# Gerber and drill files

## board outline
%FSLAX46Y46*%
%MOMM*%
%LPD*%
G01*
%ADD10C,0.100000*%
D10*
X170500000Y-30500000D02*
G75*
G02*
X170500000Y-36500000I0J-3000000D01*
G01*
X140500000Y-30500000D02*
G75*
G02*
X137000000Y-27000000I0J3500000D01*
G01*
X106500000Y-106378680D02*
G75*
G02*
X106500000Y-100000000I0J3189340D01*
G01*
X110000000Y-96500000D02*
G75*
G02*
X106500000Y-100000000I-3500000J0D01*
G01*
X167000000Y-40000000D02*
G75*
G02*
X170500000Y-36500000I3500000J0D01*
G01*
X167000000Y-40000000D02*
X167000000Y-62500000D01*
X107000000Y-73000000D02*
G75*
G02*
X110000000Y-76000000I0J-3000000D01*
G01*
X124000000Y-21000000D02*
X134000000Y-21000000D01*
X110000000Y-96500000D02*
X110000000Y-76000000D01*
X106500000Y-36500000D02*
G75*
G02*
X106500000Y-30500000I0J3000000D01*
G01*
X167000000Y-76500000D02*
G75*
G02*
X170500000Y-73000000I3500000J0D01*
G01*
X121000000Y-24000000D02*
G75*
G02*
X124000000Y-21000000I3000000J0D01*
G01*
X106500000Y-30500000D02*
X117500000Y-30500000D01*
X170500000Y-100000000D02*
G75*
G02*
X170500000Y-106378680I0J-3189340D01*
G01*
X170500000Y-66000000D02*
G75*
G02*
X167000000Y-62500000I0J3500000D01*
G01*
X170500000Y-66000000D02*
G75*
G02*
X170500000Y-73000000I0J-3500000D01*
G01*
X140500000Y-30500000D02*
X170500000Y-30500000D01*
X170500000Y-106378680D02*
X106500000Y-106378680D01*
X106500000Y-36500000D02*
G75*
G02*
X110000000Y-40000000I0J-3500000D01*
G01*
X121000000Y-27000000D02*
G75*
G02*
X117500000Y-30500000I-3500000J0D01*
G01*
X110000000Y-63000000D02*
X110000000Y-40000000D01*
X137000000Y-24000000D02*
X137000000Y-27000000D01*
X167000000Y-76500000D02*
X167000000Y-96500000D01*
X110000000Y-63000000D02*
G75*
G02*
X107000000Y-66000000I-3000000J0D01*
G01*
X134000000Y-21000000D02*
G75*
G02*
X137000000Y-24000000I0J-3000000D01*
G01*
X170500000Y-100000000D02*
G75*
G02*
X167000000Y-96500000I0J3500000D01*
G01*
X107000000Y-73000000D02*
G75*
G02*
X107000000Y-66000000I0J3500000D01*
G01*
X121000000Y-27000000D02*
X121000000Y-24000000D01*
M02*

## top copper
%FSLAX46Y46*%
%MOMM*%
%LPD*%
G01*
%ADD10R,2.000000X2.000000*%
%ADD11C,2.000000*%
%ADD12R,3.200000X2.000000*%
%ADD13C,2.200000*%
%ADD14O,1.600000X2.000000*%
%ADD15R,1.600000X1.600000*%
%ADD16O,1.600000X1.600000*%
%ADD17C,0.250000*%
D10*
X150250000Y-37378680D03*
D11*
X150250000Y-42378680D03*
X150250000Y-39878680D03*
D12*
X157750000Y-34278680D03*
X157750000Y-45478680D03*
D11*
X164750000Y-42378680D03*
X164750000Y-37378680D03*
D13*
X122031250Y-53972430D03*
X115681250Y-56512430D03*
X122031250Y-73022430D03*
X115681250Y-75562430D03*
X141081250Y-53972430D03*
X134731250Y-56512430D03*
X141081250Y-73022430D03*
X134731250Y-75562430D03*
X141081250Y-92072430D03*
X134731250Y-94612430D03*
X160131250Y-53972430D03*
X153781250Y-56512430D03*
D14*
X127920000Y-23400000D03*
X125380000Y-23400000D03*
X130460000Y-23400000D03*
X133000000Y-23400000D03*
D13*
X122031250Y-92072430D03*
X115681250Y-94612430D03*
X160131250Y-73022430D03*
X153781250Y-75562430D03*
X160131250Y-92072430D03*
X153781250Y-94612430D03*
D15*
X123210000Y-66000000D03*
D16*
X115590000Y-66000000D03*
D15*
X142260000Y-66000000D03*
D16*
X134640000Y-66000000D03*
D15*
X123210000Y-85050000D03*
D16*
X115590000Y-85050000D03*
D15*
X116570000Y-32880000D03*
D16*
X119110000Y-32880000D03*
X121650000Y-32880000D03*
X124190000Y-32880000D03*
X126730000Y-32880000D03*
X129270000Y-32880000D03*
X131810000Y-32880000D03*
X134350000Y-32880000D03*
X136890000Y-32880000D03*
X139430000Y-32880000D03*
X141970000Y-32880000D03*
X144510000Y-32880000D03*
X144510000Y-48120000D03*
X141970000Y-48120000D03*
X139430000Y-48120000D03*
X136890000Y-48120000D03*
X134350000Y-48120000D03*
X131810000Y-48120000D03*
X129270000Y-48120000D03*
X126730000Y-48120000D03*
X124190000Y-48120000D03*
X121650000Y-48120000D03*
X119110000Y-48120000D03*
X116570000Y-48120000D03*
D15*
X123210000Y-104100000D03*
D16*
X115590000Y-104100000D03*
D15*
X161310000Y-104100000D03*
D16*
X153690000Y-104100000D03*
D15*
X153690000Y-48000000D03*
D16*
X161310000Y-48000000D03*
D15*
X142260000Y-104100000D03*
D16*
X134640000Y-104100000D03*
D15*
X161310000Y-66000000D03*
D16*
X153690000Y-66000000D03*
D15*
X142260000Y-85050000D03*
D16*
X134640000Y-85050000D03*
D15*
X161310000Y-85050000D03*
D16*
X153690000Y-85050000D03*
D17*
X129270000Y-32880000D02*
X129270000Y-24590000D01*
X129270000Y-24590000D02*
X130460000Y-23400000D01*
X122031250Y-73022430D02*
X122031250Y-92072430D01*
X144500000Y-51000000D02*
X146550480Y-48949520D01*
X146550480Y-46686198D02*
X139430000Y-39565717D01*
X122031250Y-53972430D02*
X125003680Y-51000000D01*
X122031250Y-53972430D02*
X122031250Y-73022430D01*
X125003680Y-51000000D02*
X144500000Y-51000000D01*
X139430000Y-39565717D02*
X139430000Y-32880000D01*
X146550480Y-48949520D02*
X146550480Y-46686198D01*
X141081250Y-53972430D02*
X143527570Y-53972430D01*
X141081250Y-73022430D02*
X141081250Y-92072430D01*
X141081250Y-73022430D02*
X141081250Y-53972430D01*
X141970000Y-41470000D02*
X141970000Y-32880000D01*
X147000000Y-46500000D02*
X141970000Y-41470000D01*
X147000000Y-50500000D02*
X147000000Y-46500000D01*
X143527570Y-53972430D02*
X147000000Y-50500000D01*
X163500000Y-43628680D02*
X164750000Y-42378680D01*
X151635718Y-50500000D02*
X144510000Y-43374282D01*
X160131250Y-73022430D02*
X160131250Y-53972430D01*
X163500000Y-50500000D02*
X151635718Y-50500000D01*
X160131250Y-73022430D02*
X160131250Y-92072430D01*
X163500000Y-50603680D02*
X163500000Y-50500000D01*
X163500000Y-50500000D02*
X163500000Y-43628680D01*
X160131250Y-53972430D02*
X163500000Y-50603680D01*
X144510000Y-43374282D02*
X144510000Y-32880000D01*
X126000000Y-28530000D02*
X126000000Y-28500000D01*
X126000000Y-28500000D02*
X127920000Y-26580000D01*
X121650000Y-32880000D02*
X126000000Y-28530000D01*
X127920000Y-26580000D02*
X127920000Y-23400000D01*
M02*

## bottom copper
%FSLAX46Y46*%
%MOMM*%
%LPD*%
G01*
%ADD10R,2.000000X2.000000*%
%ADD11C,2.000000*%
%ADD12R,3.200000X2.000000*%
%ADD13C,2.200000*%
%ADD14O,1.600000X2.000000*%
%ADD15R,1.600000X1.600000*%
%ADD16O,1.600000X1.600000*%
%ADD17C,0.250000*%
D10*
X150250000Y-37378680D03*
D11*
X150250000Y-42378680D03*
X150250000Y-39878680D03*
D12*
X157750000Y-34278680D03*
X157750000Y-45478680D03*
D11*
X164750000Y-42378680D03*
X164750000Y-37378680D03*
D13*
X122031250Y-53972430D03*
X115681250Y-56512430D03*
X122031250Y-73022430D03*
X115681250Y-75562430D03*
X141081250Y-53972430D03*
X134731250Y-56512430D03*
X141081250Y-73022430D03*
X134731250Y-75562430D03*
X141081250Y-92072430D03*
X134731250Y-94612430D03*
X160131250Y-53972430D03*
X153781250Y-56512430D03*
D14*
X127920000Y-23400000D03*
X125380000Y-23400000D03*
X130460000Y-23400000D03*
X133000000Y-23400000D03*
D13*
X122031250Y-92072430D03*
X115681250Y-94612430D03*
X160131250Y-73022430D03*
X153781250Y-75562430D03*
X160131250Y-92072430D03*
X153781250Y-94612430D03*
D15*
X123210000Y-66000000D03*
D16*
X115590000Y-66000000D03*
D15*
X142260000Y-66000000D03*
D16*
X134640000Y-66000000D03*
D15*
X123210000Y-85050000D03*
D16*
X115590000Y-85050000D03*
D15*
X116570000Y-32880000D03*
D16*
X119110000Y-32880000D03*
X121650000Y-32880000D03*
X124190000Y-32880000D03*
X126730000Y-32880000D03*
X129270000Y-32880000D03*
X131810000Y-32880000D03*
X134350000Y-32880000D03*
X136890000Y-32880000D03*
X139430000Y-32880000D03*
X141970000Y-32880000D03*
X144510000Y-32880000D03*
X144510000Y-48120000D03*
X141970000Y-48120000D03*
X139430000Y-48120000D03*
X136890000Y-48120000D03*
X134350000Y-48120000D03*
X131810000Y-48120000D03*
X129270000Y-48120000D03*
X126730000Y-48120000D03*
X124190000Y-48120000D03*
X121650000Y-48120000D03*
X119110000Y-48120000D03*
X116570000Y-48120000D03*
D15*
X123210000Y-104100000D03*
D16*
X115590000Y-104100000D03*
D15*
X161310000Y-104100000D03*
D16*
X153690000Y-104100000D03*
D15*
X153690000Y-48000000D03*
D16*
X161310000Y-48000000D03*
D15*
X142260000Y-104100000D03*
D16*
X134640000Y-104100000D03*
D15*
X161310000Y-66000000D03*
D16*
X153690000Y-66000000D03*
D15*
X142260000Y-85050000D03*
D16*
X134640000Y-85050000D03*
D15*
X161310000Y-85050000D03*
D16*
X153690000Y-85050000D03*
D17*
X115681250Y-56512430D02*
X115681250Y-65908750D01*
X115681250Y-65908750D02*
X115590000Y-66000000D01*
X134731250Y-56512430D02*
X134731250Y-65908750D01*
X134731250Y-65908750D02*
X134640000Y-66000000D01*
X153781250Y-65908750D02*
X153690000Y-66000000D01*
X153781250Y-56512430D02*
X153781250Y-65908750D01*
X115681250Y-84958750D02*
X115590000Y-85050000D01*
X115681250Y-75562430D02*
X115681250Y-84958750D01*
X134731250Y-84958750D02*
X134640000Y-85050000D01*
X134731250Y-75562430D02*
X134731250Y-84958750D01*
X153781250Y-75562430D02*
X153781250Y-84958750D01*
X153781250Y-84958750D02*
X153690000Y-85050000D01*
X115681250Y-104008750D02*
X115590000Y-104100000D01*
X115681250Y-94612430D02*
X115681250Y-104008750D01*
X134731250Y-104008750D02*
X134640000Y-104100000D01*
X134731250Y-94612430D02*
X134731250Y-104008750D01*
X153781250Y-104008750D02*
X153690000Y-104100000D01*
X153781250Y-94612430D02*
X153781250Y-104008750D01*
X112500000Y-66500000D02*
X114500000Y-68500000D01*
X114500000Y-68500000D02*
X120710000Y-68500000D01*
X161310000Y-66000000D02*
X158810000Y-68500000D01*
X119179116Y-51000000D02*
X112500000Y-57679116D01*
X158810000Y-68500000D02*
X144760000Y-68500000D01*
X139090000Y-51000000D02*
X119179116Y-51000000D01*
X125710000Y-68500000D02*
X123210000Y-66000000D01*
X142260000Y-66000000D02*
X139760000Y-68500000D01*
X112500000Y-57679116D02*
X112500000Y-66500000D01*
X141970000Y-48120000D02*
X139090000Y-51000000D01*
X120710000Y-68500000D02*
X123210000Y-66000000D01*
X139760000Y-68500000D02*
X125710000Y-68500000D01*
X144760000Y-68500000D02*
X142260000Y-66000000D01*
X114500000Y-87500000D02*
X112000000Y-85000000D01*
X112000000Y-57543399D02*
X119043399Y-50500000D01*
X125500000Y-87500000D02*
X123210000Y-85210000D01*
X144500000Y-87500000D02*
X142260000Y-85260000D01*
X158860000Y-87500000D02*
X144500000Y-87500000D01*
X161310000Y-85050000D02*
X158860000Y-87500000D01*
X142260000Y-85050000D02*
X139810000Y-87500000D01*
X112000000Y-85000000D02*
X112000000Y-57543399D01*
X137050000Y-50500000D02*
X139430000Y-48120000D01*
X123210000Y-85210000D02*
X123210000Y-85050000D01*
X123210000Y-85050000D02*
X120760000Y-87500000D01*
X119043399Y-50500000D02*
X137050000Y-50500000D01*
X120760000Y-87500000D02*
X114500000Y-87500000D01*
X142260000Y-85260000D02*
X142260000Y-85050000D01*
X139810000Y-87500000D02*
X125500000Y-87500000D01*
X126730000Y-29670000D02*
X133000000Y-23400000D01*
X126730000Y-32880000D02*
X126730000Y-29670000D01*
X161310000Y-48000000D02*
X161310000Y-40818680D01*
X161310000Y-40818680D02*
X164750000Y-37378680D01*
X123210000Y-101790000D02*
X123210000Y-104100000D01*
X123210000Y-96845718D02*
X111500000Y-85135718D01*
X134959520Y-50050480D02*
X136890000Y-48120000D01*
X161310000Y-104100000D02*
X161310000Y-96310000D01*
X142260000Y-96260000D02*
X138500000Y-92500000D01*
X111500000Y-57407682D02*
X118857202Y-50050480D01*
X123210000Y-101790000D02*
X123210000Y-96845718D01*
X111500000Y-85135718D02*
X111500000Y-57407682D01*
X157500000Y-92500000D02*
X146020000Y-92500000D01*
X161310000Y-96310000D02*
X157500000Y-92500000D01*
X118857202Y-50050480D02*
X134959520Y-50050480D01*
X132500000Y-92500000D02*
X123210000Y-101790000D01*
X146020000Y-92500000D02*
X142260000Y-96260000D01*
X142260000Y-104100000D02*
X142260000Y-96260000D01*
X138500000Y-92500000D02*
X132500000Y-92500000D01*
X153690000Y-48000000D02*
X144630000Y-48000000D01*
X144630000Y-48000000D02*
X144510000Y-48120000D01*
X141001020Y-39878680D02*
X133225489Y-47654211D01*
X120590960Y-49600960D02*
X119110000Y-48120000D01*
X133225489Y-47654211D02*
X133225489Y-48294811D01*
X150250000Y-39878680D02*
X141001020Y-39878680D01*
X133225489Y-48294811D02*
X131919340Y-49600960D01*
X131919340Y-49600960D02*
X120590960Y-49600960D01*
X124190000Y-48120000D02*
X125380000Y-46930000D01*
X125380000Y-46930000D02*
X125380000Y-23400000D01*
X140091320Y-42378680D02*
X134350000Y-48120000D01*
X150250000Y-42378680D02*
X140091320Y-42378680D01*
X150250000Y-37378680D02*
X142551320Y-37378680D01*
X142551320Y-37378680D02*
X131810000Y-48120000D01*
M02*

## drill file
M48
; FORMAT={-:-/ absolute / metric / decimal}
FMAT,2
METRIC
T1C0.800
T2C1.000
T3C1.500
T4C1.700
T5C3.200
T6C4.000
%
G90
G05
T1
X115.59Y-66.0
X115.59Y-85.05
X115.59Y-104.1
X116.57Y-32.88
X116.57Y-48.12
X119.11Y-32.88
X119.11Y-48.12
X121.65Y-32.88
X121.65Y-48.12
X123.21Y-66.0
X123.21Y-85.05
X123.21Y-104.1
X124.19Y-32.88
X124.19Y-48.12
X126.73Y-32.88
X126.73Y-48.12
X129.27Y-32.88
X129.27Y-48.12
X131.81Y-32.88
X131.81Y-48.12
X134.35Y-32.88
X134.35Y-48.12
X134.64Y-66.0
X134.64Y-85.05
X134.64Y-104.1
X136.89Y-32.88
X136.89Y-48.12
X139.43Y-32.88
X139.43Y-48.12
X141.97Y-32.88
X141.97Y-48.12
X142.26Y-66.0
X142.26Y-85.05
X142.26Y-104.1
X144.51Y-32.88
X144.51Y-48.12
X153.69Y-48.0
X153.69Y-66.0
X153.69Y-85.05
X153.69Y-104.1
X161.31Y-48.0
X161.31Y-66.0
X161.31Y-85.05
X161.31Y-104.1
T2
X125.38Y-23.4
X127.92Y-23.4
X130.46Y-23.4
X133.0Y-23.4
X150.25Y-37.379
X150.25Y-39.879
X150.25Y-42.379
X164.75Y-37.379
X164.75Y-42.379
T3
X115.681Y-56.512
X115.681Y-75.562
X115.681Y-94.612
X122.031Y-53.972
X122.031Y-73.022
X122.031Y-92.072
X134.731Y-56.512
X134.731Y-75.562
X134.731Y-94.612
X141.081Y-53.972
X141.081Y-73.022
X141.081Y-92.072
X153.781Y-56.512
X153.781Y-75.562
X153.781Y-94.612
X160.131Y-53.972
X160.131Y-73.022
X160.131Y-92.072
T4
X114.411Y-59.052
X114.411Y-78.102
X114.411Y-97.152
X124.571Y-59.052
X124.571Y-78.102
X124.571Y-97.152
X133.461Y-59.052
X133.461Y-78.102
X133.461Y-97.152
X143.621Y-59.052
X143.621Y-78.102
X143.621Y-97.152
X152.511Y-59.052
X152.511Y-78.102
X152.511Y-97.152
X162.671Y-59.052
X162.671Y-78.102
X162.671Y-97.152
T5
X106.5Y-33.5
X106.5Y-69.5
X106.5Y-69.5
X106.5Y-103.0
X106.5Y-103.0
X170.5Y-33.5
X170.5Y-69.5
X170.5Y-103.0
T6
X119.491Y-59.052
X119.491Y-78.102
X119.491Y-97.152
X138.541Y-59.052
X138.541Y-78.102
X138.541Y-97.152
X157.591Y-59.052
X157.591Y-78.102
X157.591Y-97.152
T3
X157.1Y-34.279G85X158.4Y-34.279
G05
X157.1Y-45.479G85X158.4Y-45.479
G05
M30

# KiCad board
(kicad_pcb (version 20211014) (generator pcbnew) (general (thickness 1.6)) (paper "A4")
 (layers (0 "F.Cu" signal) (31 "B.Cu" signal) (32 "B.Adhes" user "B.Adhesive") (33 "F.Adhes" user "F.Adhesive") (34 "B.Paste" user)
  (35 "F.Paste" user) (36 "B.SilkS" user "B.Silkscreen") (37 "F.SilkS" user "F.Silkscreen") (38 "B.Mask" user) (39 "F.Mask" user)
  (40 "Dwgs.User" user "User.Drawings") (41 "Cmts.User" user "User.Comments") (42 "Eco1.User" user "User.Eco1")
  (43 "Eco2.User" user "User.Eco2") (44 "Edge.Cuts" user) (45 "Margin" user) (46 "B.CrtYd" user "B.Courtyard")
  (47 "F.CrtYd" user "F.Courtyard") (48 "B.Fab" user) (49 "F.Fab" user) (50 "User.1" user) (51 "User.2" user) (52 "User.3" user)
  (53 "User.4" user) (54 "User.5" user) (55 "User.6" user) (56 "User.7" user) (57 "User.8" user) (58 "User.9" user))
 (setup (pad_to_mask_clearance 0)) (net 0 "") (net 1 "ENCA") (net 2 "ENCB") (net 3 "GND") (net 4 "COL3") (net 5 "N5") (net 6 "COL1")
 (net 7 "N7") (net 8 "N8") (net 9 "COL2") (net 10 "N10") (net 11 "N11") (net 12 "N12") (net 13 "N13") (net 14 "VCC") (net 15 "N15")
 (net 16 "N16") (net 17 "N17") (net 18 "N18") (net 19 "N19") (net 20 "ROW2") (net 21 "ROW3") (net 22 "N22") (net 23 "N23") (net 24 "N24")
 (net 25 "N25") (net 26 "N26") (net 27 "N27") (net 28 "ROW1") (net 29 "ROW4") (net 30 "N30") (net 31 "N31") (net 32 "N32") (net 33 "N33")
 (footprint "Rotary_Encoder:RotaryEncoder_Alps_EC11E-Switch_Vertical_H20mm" (layer "F.Cu") (at 150.25 37.37868)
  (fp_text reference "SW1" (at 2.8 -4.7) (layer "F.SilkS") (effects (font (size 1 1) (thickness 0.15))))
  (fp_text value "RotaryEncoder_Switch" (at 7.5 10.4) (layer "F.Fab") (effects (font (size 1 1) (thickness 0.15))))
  (pad "A" thru_hole rect (at 0 0) (size 2 2) (drill 1) (layers *.Cu *.Mask) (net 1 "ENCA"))
  (pad "B" thru_hole circle (at 0 5) (size 2 2) (drill 1) (layers *.Cu *.Mask) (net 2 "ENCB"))
  (pad "C" thru_hole circle (at 0 2.5) (size 2 2) (drill 1) (layers *.Cu *.Mask) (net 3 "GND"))
  (pad "MP" thru_hole rect (at 7.5 -3.1) (size 3.2 2) (drill oval 2.8 1.5) (layers *.Cu *.Mask))
  (pad "MP" thru_hole rect (at 7.5 8.1) (size 3.2 2) (drill oval 2.8 1.5) (layers *.Cu *.Mask))
  (pad "S1" thru_hole circle (at 14.5 5) (size 2 2) (drill 1) (layers *.Cu *.Mask) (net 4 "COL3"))
  (pad "S2" thru_hole circle (at 14.5 0) (size 2 2) (drill 1) (layers *.Cu *.Mask) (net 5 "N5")))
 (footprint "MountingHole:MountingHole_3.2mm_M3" (layer "F.Cu") (at 106.5 69.5)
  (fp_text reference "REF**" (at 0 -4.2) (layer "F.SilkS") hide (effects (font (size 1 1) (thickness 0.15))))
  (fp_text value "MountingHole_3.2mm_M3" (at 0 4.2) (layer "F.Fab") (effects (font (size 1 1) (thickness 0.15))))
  (pad "" np_thru_hole circle (at 0 0) (size 3.2 3.2) (drill 3.2) (layers *.Cu *.Mask)))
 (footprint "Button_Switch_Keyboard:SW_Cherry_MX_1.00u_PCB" (layer "F.Cu") (at 122.03125 53.97243)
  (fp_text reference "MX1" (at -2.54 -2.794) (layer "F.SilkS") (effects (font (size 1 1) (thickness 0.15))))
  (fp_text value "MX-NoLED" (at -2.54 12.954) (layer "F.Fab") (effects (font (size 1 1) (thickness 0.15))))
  (pad "" np_thru_hole circle (at -7.62 5.08) (size 1.7 1.7) (drill 1.7) (layers *.Cu *.Mask))
  (pad "" np_thru_hole circle (at 2.54 5.08) (size 1.7 1.7) (drill 1.7) (layers *.Cu *.Mask))
  (pad "" np_thru_hole circle (at -2.54 5.08) (size 4 4) (drill 4) (layers *.Cu *.Mask))
  (pad "1" thru_hole circle (at 0 0) (size 2.2 2.2) (drill 1.5) (layers *.Cu *.Mask) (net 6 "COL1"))
  (pad "2" thru_hole circle (at -6.35 2.54) (size 2.2 2.2) (drill 1.5) (layers *.Cu *.Mask) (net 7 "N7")))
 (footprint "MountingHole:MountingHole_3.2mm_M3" (layer "F.Cu") (at 170.5 103)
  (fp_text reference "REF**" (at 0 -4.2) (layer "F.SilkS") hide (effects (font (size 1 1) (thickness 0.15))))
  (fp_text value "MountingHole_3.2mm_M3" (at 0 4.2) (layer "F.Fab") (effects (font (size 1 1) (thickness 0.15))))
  (pad "" np_thru_hole circle (at 0 0) (size 3.2 3.2) (drill 3.2) (layers *.Cu *.Mask)))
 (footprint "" (layer "F.Cu") (at 106.5 103)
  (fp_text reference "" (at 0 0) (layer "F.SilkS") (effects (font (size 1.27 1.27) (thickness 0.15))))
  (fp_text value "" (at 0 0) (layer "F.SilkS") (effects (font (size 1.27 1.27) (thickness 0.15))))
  (pad "" np_thru_hole circle (at 0 0) (size 3.2 3.2) (drill 3.2) (layers *.Cu *.Mask)))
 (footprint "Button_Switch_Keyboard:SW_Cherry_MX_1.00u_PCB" (layer "F.Cu") (at 122.03125 73.02243)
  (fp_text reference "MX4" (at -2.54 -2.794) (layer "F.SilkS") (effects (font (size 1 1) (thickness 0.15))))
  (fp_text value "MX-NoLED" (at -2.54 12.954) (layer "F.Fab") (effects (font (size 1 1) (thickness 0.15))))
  (pad "" np_thru_hole circle (at -2.54 5.08) (size 4 4) (drill 4) (layers *.Cu *.Mask))
  (pad "" np_thru_hole circle (at -7.62 5.08) (size 1.7 1.7) (drill 1.7) (layers *.Cu *.Mask))
  (pad "" np_thru_hole circle (at 2.54 5.08) (size 1.7 1.7) (drill 1.7) (layers *.Cu *.Mask))
  (pad "1" thru_hole circle (at 0 0) (size 2.2 2.2) (drill 1.5) (layers *.Cu *.Mask) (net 6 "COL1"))
  (pad "2" thru_hole circle (at -6.35 2.54) (size 2.2 2.2) (drill 1.5) (layers *.Cu *.Mask) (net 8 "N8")))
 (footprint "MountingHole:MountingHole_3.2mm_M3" (layer "F.Cu") (at 106.5 103)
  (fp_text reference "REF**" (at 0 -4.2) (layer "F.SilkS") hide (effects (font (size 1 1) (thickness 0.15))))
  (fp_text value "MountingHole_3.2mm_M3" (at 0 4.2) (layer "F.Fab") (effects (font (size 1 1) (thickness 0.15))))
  (pad "" np_thru_hole circle (at 0 0) (size 3.2 3.2) (drill 3.2) (layers *.Cu *.Mask)))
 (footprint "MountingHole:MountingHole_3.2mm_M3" (layer "F.Cu") (at 170.5 69.5)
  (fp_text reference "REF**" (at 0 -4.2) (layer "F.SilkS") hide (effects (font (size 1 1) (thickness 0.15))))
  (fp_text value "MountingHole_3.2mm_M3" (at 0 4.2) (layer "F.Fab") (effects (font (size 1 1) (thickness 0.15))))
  (pad "" np_thru_hole circle (at 0 0) (size 3.2 3.2) (drill 3.2) (layers *.Cu *.Mask)))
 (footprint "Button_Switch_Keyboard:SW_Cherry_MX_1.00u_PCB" (layer "F.Cu") (at 141.08125 53.97243)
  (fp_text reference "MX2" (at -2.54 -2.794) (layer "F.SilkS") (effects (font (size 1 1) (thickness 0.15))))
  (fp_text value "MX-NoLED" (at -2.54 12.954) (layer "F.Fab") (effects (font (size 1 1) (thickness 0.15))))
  (pad "" np_thru_hole circle (at -2.54 5.08) (size 4 4) (drill 4) (layers *.Cu *.Mask))
  (pad "" np_thru_hole circle (at -7.62 5.08) (size 1.7 1.7) (drill 1.7) (layers *.Cu *.Mask))
  (pad "" np_thru_hole circle (at 2.54 5.08) (size 1.7 1.7) (drill 1.7) (layers *.Cu *.Mask))
  (pad "1" thru_hole circle (at 0 0) (size 2.2 2.2) (drill 1.5) (layers *.Cu *.Mask) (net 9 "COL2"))
  (pad "2" thru_hole circle (at -6.35 2.54) (size 2.2 2.2) (drill 1.5) (layers *.Cu *.Mask) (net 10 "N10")))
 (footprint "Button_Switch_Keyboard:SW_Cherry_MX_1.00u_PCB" (layer "F.Cu") (at 141.08125 73.02243)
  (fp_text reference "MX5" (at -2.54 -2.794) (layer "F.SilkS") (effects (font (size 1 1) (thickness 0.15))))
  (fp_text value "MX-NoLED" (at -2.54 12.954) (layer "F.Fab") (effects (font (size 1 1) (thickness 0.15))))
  (pad "" np_thru_hole circle (at -2.54 5.08) (size 4 4) (drill 4) (layers *.Cu *.Mask))
  (pad "" np_thru_hole circle (at 2.54 5.08) (size 1.7 1.7) (drill 1.7) (layers *.Cu *.Mask))
  (pad "" np_thru_hole circle (at -7.62 5.08) (size 1.7 1.7) (drill 1.7) (layers *.Cu *.Mask))
  (pad "1" thru_hole circle (at 0 0) (size 2.2 2.2) (drill 1.5) (layers *.Cu *.Mask) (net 9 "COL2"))
  (pad "2" thru_hole circle (at -6.35 2.54) (size 2.2 2.2) (drill 1.5) (layers *.Cu *.Mask) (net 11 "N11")))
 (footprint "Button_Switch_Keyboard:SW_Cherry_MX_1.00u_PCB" (layer "F.Cu") (at 141.08125 92.07243)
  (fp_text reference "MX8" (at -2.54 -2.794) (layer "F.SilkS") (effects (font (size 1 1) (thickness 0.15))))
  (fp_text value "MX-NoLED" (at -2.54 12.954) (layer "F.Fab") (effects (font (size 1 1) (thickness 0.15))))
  (pad "" np_thru_hole circle (at -2.54 5.08) (size 4 4) (drill 4) (layers *.Cu *.Mask))
  (pad "" np_thru_hole circle (at -7.62 5.08) (size 1.7 1.7) (drill 1.7) (layers *.Cu *.Mask))
  (pad "" np_thru_hole circle (at 2.54 5.08) (size 1.7 1.7) (drill 1.7) (layers *.Cu *.Mask))
  (pad "1" thru_hole circle (at 0 0) (size 2.2 2.2) (drill 1.5) (layers *.Cu *.Mask) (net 9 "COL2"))
  (pad "2" thru_hole circle (at -6.35 2.54) (size 2.2 2.2) (drill 1.5) (layers *.Cu *.Mask) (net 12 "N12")))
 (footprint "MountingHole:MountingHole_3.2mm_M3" (layer "F.Cu") (at 106.5 33.5)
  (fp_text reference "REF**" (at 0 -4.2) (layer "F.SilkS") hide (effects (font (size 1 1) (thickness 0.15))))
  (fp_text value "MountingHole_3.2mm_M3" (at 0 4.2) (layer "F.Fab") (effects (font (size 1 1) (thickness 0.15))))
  (pad "" np_thru_hole circle (at 0 0) (size 3.2 3.2) (drill 3.2) (layers *.Cu *.Mask)))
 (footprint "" (layer "F.Cu") (at 106.5 69.5)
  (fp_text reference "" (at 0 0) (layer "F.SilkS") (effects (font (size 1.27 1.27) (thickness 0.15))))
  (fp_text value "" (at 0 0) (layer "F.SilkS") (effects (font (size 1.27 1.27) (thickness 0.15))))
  (pad "" np_thru_hole circle (at 0 0) (size 3.2 3.2) (drill 3.2) (layers *.Cu *.Mask)))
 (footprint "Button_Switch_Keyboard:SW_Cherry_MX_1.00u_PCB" (layer "F.Cu") (at 160.13125 53.97243)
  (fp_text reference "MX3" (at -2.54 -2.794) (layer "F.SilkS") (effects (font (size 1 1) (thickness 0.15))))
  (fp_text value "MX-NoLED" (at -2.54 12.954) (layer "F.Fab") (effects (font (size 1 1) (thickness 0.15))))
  (pad "" np_thru_hole circle (at 2.54 5.08) (size 1.7 1.7) (drill 1.7) (layers *.Cu *.Mask))
  (pad "" np_thru_hole circle (at -2.54 5.08) (size 4 4) (drill 4) (layers *.Cu *.Mask))
  (pad "" np_thru_hole circle (at -7.62 5.08) (size 1.7 1.7) (drill 1.7) (layers *.Cu *.Mask))
  (pad "1" thru_hole circle (at 0 0) (size 2.2 2.2) (drill 1.5) (layers *.Cu *.Mask) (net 4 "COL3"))
  (pad "2" thru_hole circle (at -6.35 2.54) (size 2.2 2.2) (drill 1.5) (layers *.Cu *.Mask) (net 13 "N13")))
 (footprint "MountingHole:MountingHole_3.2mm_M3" (layer "F.Cu") (at 170.5 33.5)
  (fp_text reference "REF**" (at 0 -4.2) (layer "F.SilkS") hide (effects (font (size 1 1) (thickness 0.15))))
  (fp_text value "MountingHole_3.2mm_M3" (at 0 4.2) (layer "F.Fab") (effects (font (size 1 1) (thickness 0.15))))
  (pad "" np_thru_hole circle (at 0 0) (size 3.2 3.2) (drill 3.2) (layers *.Cu *.Mask)))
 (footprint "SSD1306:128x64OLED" (layer "F.Cu") (at 129 34)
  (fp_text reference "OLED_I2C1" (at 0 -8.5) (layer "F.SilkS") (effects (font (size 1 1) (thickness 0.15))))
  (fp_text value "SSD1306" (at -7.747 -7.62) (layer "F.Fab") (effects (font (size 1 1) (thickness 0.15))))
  (pad "1" thru_hole oval (at -1.08 -10.6 90) (size 2 1.6) (drill 1) (layers *.Cu *.Mask) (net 3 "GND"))
  (pad "2" thru_hole oval (at -3.62 -10.6 90) (size 2 1.6) (drill 1) (layers *.Cu *.Mask) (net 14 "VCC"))
  (pad "3" thru_hole oval (at 1.46 -10.6 90) (size 2 1.6) (drill 1) (layers *.Cu *.Mask) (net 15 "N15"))
  (pad "4" thru_hole oval (at 4 -10.6 90) (size 2 1.6) (drill 1) (layers *.Cu *.Mask) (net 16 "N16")))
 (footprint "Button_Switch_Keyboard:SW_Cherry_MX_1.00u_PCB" (layer "F.Cu") (at 122.03125 92.07243)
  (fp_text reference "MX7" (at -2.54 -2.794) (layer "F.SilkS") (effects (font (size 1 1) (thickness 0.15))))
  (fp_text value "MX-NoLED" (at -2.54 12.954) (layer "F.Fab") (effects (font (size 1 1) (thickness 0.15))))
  (pad "" np_thru_hole circle (at -7.62 5.08) (size 1.7 1.7) (drill 1.7) (layers *.Cu *.Mask))
  (pad "" np_thru_hole circle (at -2.54 5.08) (size 4 4) (drill 4) (layers *.Cu *.Mask))
  (pad "" np_thru_hole circle (at 2.54 5.08) (size 1.7 1.7) (drill 1.7) (layers *.Cu *.Mask))
  (pad "1" thru_hole circle (at 0 0) (size 2.2 2.2) (drill 1.5) (layers *.Cu *.Mask) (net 6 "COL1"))
  (pad "2" thru_hole circle (at -6.35 2.54) (size 2.2 2.2) (drill 1.5) (layers *.Cu *.Mask) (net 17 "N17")))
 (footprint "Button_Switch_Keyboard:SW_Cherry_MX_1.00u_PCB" (layer "F.Cu") (at 160.13125 73.02243)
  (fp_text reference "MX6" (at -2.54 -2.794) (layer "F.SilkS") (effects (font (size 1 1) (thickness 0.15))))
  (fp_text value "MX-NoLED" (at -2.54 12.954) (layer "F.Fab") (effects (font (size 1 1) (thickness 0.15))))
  (pad "" np_thru_hole circle (at -7.62 5.08) (size 1.7 1.7) (drill 1.7) (layers *.Cu *.Mask))
  (pad "" np_thru_hole circle (at -2.54 5.08) (size 4 4) (drill 4) (layers *.Cu *.Mask))
  (pad "" np_thru_hole circle (at 2.54 5.08) (size 1.7 1.7) (drill 1.7) (layers *.Cu *.Mask))
  (pad "1" thru_hole circle (at 0 0) (size 2.2 2.2) (drill 1.5) (layers *.Cu *.Mask) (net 4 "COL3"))
  (pad "2" thru_hole circle (at -6.35 2.54) (size 2.2 2.2) (drill 1.5) (layers *.Cu *.Mask) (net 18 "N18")))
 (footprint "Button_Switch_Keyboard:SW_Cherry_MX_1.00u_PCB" (layer "F.Cu") (at 160.13125 92.07243)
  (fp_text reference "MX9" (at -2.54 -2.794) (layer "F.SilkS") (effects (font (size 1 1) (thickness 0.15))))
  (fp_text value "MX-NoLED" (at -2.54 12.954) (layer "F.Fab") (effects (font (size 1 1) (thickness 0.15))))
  (pad "" np_thru_hole circle (at -7.62 5.08) (size 1.7 1.7) (drill 1.7) (layers *.Cu *.Mask))
  (pad "" np_thru_hole circle (at 2.54 5.08) (size 1.7 1.7) (drill 1.7) (layers *.Cu *.Mask))
  (pad "" np_thru_hole circle (at -2.54 5.08) (size 4 4) (drill 4) (layers *.Cu *.Mask))
  (pad "1" thru_hole circle (at 0 0) (size 2.2 2.2) (drill 1.5) (layers *.Cu *.Mask) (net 4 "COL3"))
  (pad "2" thru_hole circle (at -6.35 2.54) (size 2.2 2.2) (drill 1.5) (layers *.Cu *.Mask) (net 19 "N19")))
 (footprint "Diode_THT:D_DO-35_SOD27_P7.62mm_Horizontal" (layer "B.Cu") (at 123.21 66 180)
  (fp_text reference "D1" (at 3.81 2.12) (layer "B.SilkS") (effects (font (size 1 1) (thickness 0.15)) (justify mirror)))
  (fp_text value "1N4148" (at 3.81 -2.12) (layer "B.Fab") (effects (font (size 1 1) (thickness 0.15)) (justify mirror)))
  (pad "1" thru_hole rect (at 0 0 180) (size 1.6 1.6) (drill 0.8) (layers *.Cu *.Mask) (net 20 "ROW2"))
  (pad "2" thru_hole oval (at 7.62 0 180) (size 1.6 1.6) (drill 0.8) (layers *.Cu *.Mask) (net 7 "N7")))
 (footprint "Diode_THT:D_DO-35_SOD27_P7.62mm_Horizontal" (layer "B.Cu") (at 142.26 66 180)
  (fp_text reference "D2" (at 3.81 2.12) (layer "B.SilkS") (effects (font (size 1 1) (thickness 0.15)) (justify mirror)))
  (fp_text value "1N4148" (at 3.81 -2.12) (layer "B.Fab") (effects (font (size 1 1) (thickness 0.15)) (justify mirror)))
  (pad "1" thru_hole rect (at 0 0 180) (size 1.6 1.6) (drill 0.8) (layers *.Cu *.Mask) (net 20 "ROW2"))
  (pad "2" thru_hole oval (at 7.62 0 180) (size 1.6 1.6) (drill 0.8) (layers *.Cu *.Mask) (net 10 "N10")))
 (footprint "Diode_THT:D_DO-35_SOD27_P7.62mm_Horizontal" (layer "B.Cu") (at 123.21 85.05 180)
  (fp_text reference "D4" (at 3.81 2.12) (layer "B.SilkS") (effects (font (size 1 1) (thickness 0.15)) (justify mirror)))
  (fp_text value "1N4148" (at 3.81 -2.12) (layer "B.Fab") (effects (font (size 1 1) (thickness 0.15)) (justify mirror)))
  (pad "1" thru_hole rect (at 0 0 180) (size 1.6 1.6) (drill 0.8) (layers *.Cu *.Mask) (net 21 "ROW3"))
  (pad "2" thru_hole oval (at 7.62 0 180) (size 1.6 1.6) (drill 0.8) (layers *.Cu *.Mask) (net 8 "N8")))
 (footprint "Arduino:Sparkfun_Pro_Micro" (layer "B.Cu") (at 144.51 48.12 90)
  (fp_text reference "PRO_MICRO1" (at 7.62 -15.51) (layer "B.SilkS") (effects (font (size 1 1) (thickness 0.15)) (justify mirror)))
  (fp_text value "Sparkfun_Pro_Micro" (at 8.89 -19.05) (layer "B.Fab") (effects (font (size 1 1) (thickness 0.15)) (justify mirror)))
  (pad "1" thru_hole rect (at 15.24 -27.94 90) (size 1.6 1.6) (drill 0.8) (layers *.Cu *.Mask) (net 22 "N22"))
  (pad "2" thru_hole oval (at 15.24 -25.4 90) (size 1.6 1.6) (drill 0.8) (layers *.Cu *.Mask) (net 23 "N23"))
  (pad "3" thru_hole oval (at 15.24 -22.86 90) (size 1.6 1.6) (drill 0.8) (layers *.Cu *.Mask) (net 3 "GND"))
  (pad "4" thru_hole oval (at 15.24 -20.32 90) (size 1.6 1.6) (drill 0.8) (layers *.Cu *.Mask) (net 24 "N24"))
  (pad "5" thru_hole oval (at 15.24 -17.78 90) (size 1.6 1.6) (drill 0.8) (layers *.Cu *.Mask) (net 16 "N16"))
  (pad "6" thru_hole oval (at 15.24 -15.24 90) (size 1.6 1.6) (drill 0.8) (layers *.Cu *.Mask) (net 15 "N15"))
  (pad "7" thru_hole oval (at 15.24 -12.7 90) (size 1.6 1.6) (drill 0.8) (layers *.Cu *.Mask) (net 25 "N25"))
  (pad "8" thru_hole oval (at 15.24 -10.16 90) (size 1.6 1.6) (drill 0.8) (layers *.Cu *.Mask) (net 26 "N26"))
  (pad "9" thru_hole oval (at 15.24 -7.62 90) (size 1.6 1.6) (drill 0.8) (layers *.Cu *.Mask) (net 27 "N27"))
  (pad "10" thru_hole oval (at 15.24 -5.08 90) (size 1.6 1.6) (drill 0.8) (layers *.Cu *.Mask) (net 6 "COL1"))
  (pad "11" thru_hole oval (at 15.24 -2.54 90) (size 1.6 1.6) (drill 0.8) (layers *.Cu *.Mask) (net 9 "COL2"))
  (pad "12" thru_hole oval (at 15.24 0 90) (size 1.6 1.6) (drill 0.8) (layers *.Cu *.Mask) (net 4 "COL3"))
  (pad "13" thru_hole oval (at 0 0 90) (size 1.6 1.6) (drill 0.8) (layers *.Cu *.Mask) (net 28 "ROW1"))
  (pad "14" thru_hole oval (at 0 -2.54 90) (size 1.6 1.6) (drill 0.8) (layers *.Cu *.Mask) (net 20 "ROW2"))
  (pad "15" thru_hole oval (at 0 -5.08 90) (size 1.6 1.6) (drill 0.8) (layers *.Cu *.Mask) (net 21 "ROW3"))
  (pad "16" thru_hole oval (at 0 -7.62 90) (size 1.6 1.6) (drill 0.8) (layers *.Cu *.Mask) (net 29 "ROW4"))
  (pad "17" thru_hole oval (at 0 -10.16 90) (size 1.6 1.6) (drill 0.8) (layers *.Cu *.Mask) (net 2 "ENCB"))
  (pad "18" thru_hole oval (at 0 -12.7 90) (size 1.6 1.6) (drill 0.8) (layers *.Cu *.Mask) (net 1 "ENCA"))
  (pad "19" thru_hole oval (at 0 -15.24 90) (size 1.6 1.6) (drill 0.8) (layers *.Cu *.Mask) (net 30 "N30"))
  (pad "20" thru_hole oval (at 0 -17.78 90) (size 1.6 1.6) (drill 0.8) (layers *.Cu *.Mask) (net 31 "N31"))
  (pad "21" thru_hole oval (at 0 -20.32 90) (size 1.6 1.6) (drill 0.8) (layers *.Cu *.Mask) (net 14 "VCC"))
  (pad "22" thru_hole oval (at 0 -22.86 90) (size 1.6 1.6) (drill 0.8) (layers *.Cu *.Mask) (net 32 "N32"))
  (pad "23" thru_hole oval (at 0 -25.4 90) (size 1.6 1.6) (drill 0.8) (layers *.Cu *.Mask) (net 3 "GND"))
  (pad "24" thru_hole oval (at 0 -27.94 90) (size 1.6 1.6) (drill 0.8) (layers *.Cu *.Mask) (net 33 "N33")))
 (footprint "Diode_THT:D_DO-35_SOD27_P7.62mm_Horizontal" (layer "B.Cu") (at 123.21 104.1 180)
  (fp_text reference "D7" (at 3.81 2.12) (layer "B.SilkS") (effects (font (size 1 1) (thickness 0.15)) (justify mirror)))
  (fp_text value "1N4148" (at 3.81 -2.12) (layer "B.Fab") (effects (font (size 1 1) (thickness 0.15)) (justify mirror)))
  (pad "1" thru_hole rect (at 0 0 180) (size 1.6 1.6) (drill 0.8) (layers *.Cu *.Mask) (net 29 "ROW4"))
  (pad "2" thru_hole oval (at 7.62 0 180) (size 1.6 1.6) (drill 0.8) (layers *.Cu *.Mask) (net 17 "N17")))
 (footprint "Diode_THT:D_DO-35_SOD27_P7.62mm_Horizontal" (layer "B.Cu") (at 161.31 104.1 180)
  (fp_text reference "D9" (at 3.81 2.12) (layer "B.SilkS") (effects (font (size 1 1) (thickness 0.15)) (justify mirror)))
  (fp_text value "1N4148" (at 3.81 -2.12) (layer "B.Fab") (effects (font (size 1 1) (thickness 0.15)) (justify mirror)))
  (pad "1" thru_hole rect (at 0 0 180) (size 1.6 1.6) (drill 0.8) (layers *.Cu *.Mask) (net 29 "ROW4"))
  (pad "2" thru_hole oval (at 7.62 0 180) (size 1.6 1.6) (drill 0.8) (layers *.Cu *.Mask) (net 19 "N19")))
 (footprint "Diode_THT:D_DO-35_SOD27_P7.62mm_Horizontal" (layer "B.Cu") (at 153.69 48)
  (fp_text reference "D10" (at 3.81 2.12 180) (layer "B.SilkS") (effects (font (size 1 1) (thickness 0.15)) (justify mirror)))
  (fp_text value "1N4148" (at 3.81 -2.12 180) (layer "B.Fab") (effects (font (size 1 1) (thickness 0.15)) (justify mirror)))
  (pad "1" thru_hole rect (at 0 0) (size 1.6 1.6) (drill 0.8) (layers *.Cu *.Mask) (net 28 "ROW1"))
  (pad "2" thru_hole oval (at 7.62 0) (size 1.6 1.6) (drill 0.8) (layers *.Cu *.Mask) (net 5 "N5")))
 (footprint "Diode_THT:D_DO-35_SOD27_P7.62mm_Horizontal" (layer "B.Cu") (at 142.26 104.1 180)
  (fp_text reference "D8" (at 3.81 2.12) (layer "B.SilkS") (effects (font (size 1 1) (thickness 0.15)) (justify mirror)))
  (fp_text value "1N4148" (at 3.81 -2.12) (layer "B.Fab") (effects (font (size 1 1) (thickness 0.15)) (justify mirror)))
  (pad "1" thru_hole rect (at 0 0 180) (size 1.6 1.6) (drill 0.8) (layers *.Cu *.Mask) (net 29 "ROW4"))
  (pad "2" thru_hole oval (at 7.62 0 180) (size 1.6 1.6) (drill 0.8) (layers *.Cu *.Mask) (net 12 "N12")))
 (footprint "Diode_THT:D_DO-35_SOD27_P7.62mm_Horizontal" (layer "B.Cu") (at 161.31 66 180)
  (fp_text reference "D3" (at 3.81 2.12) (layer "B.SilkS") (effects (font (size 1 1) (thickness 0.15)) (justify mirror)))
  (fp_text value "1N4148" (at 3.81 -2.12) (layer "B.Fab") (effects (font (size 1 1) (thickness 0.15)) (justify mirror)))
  (pad "1" thru_hole rect (at 0 0 180) (size 1.6 1.6) (drill 0.8) (layers *.Cu *.Mask) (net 20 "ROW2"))
  (pad "2" thru_hole oval (at 7.62 0 180) (size 1.6 1.6) (drill 0.8) (layers *.Cu *.Mask) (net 13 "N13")))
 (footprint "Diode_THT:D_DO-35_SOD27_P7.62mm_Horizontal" (layer "B.Cu") (at 142.26 85.05 180)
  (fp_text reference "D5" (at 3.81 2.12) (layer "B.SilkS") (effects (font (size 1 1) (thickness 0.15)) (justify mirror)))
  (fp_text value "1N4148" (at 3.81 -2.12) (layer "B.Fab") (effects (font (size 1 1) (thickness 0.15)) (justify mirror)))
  (pad "1" thru_hole rect (at 0 0 180) (size 1.6 1.6) (drill 0.8) (layers *.Cu *.Mask) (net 21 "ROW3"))
  (pad "2" thru_hole oval (at 7.62 0 180) (size 1.6 1.6) (drill 0.8) (layers *.Cu *.Mask) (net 11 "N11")))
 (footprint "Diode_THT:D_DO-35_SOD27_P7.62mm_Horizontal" (layer "B.Cu") (at 161.31 85.05 180)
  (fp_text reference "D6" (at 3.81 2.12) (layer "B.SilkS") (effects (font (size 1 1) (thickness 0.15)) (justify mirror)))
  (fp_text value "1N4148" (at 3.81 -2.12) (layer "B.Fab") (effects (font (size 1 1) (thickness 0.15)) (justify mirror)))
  (pad "1" thru_hole rect (at 0 0 180) (size 1.6 1.6) (drill 0.8) (layers *.Cu *.Mask) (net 21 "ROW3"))
  (pad "2" thru_hole oval (at 7.62 0 180) (size 1.6 1.6) (drill 0.8) (layers *.Cu *.Mask) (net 18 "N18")))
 (gr_arc (start 170.5 30.5) (mid 173.5 33.5) (end 170.5 36.5) (layer "Edge.Cuts") (width 0.1))
 (gr_arc (start 140.5 30.5) (mid 138.025126 29.474874) (end 137 27) (layer "Edge.Cuts") (width 0.1))
 (gr_arc (start 106.5 106.37868) (mid 103.31066 103.18934) (end 106.5 100) (layer "Edge.Cuts") (width 0.1))
 (gr_arc (start 110 96.5) (mid 108.974874 98.974874) (end 106.5 100) (layer "Edge.Cuts") (width 0.1))
 (gr_arc (start 167 40) (mid 168.025126 37.525126) (end 170.5 36.5) (layer "Edge.Cuts") (width 0.1))
 (gr_line (start 167 40) (end 167 62.5) (layer "Edge.Cuts") (width 0.1))
 (gr_arc (start 107 73) (mid 109.12132 73.87868) (end 110 76) (layer "Edge.Cuts") (width 0.1))
 (gr_line (start 124 21) (end 134 21) (layer "Edge.Cuts") (width 0.1))
 (gr_line (start 110 96.5) (end 110 76) (layer "Edge.Cuts") (width 0.1))
 (gr_arc (start 106.5 36.5) (mid 103.5 33.5) (end 106.5 30.5) (layer "Edge.Cuts") (width 0.1))
 (gr_arc (start 167 76.5) (mid 168.025126 74.025126) (end 170.5 73) (layer "Edge.Cuts") (width 0.1))
 (gr_arc (start 121 24) (mid 121.87868 21.87868) (end 124 21) (layer "Edge.Cuts") (width 0.1))
 (gr_line (start 106.5 30.5) (end 117.5 30.5) (layer "Edge.Cuts") (width 0.1))
 (gr_arc (start 170.5 100) (mid 173.68934 103.18934) (end 170.5 106.37868) (layer "Edge.Cuts") (width 0.1))
 (gr_arc (start 170.5 66) (mid 168.025126 64.974874) (end 167 62.5) (layer "Edge.Cuts") (width 0.1))
 (gr_arc (start 170.5 66) (mid 174 69.5) (end 170.5 73) (layer "Edge.Cuts") (width 0.1))
 (gr_line (start 140.5 30.5) (end 170.5 30.5) (layer "Edge.Cuts") (width 0.1))
 (gr_line (start 170.5 106.37868) (end 106.5 106.37868) (layer "Edge.Cuts") (width 0.1))
 (gr_arc (start 106.5 36.5) (mid 108.974874 37.525126) (end 110 40) (layer "Edge.Cuts") (width 0.1))
 (gr_arc (start 121 27) (mid 119.974874 29.474874) (end 117.5 30.5) (layer "Edge.Cuts") (width 0.1))
 (gr_line (start 110 63) (end 110 40) (layer "Edge.Cuts") (width 0.1))
 (gr_line (start 137 24) (end 137 27) (layer "Edge.Cuts") (width 0.1))
 (gr_line (start 167 76.5) (end 167 96.5) (layer "Edge.Cuts") (width 0.1))
 (gr_arc (start 110 63) (mid 109.12132 65.12132) (end 107 66) (layer "Edge.Cuts") (width 0.1))
 (gr_arc (start 134 21) (mid 136.12132 21.87868) (end 137 24) (layer "Edge.Cuts") (width 0.1))
 (gr_arc (start 170.5 100) (mid 168.025126 98.974874) (end 167 96.5) (layer "Edge.Cuts") (width 0.1))
 (gr_arc (start 107 73) (mid 103.5 69.5) (end 107 66) (layer "Edge.Cuts") (width 0.1))
 (gr_line (start 121 27) (end 121 24) (layer "Edge.Cuts") (width 0.1))
 (segment (start 115.68125 56.51243) (end 115.68125 65.90875) (width 0.25) (layer "B.Cu") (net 7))
 (segment (start 115.68125 65.90875) (end 115.59 66) (width 0.25) (layer "B.Cu") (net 7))
 (segment (start 134.73125 56.51243) (end 134.73125 65.90875) (width 0.25) (layer "B.Cu") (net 10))
 (segment (start 134.73125 65.90875) (end 134.64 66) (width 0.25) (layer "B.Cu") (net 10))
 (segment (start 153.78125 65.90875) (end 153.69 66) (width 0.25) (layer "B.Cu") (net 13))
 (segment (start 153.78125 56.51243) (end 153.78125 65.90875) (width 0.25) (layer "B.Cu") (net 13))
 (segment (start 115.68125 84.95875) (end 115.59 85.05) (width 0.25) (layer "B.Cu") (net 8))
 (segment (start 115.68125 75.56243) (end 115.68125 84.95875) (width 0.25) (layer "B.Cu") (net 8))
 (segment (start 134.73125 84.95875) (end 134.64 85.05) (width 0.25) (layer "B.Cu") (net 11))
 (segment (start 134.73125 75.56243) (end 134.73125 84.95875) (width 0.25) (layer "B.Cu") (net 11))
 (segment (start 153.78125 75.56243) (end 153.78125 84.95875) (width 0.25) (layer "B.Cu") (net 18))
 (segment (start 153.78125 84.95875) (end 153.69 85.05) (width 0.25) (layer "B.Cu") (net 18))
 (segment (start 115.68125 104.00875) (end 115.59 104.1) (width 0.25) (layer "B.Cu") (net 17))
 (segment (start 115.68125 94.61243) (end 115.68125 104.00875) (width 0.25) (layer "B.Cu") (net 17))
 (segment (start 134.73125 104.00875) (end 134.64 104.1) (width 0.25) (layer "B.Cu") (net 12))
 (segment (start 134.73125 94.61243) (end 134.73125 104.00875) (width 0.25) (layer "B.Cu") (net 12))
 (segment (start 153.78125 104.00875) (end 153.69 104.1) (width 0.25) (layer "B.Cu") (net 19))
 (segment (start 153.78125 94.61243) (end 153.78125 104.00875) (width 0.25) (layer "B.Cu") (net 19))
 (segment (start 112.5 66.5) (end 114.5 68.5) (width 0.25) (layer "B.Cu") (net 20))
 (segment (start 114.5 68.5) (end 120.71 68.5) (width 0.25) (layer "B.Cu") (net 20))
 (segment (start 161.31 66) (end 158.81 68.5) (width 0.25) (layer "B.Cu") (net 20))
 (segment (start 119.179116 51) (end 112.5 57.679116) (width 0.25) (layer "B.Cu") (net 20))
 (segment (start 158.81 68.5) (end 144.76 68.5) (width 0.25) (layer "B.Cu") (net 20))
 (segment (start 139.09 51) (end 119.179116 51) (width 0.25) (layer "B.Cu") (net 20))
 (segment (start 125.71 68.5) (end 123.21 66) (width 0.25) (layer "B.Cu") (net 20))
 (segment (start 142.26 66) (end 139.76 68.5) (width 0.25) (layer "B.Cu") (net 20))
 (segment (start 112.5 57.679116) (end 112.5 66.5) (width 0.25) (layer "B.Cu") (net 20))
 (segment (start 141.97 48.12) (end 139.09 51) (width 0.25) (layer "B.Cu") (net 20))
 (segment (start 120.71 68.5) (end 123.21 66) (width 0.25) (layer "B.Cu") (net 20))
 (segment (start 139.76 68.5) (end 125.71 68.5) (width 0.25) (layer "B.Cu") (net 20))
 (segment (start 144.76 68.5) (end 142.26 66) (width 0.25) (layer "B.Cu") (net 20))
 (segment (start 114.5 87.5) (end 112 85) (width 0.25) (layer "B.Cu") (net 21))
 (segment (start 112 57.543399) (end 119.043399 50.5) (width 0.25) (layer "B.Cu") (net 21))
 (segment (start 125.5 87.5) (end 123.21 85.21) (width 0.25) (layer "B.Cu") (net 21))
 (segment (start 144.5 87.5) (end 142.26 85.26) (width 0.25) (layer "B.Cu") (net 21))
 (segment (start 158.86 87.5) (end 144.5 87.5) (width 0.25) (layer "B.Cu") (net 21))
 (segment (start 161.31 85.05) (end 158.86 87.5) (width 0.25) (layer "B.Cu") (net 21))
 (segment (start 142.26 85.05) (end 139.81 87.5) (width 0.25) (layer "B.Cu") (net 21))
 (segment (start 112 85) (end 112 57.543399) (width 0.25) (layer "B.Cu") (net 21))
 (segment (start 137.05 50.5) (end 139.43 48.12) (width 0.25) (layer "B.Cu") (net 21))
 (segment (start 123.21 85.21) (end 123.21 85.05) (width 0.25) (layer "B.Cu") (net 21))
 (segment (start 123.21 85.05) (end 120.76 87.5) (width 0.25) (layer "B.Cu") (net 21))
 (segment (start 119.043399 50.5) (end 137.05 50.5) (width 0.25) (layer "B.Cu") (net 21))
 (segment (start 120.76 87.5) (end 114.5 87.5) (width 0.25) (layer "B.Cu") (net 21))
 (segment (start 142.26 85.26) (end 142.26 85.05) (width 0.25) (layer "B.Cu") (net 21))
 (segment (start 139.81 87.5) (end 125.5 87.5) (width 0.25) (layer "B.Cu") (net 21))
 (segment (start 129.27 32.88) (end 129.27 24.59) (width 0.25) (layer "F.Cu") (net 15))
 (segment (start 129.27 24.59) (end 130.46 23.4) (width 0.25) (layer "F.Cu") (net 15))
 (segment (start 126.73 29.67) (end 133 23.4) (width 0.25) (layer "B.Cu") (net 16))
 (segment (start 126.73 32.88) (end 126.73 29.67) (width 0.25) (layer "B.Cu") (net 16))
 (segment (start 161.31 48) (end 161.31 40.81868) (width 0.25) (layer "B.Cu") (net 5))
 (segment (start 161.31 40.81868) (end 164.75 37.37868) (width 0.25) (layer "B.Cu") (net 5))
 (segment (start 123.21 101.79) (end 123.21 104.1) (width 0.25) (layer "B.Cu") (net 29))
 (segment (start 123.21 96.845718) (end 111.5 85.135718) (width 0.25) (layer "B.Cu") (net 29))
 (segment (start 134.95952 50.05048) (end 136.89 48.12) (width 0.25) (layer "B.Cu") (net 29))
 (segment (start 161.31 104.1) (end 161.31 96.31) (width 0.25) (layer "B.Cu") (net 29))
 (segment (start 142.26 96.26) (end 138.5 92.5) (width 0.25) (layer "B.Cu") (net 29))
 (segment (start 111.5 57.407682) (end 118.857202 50.05048) (width 0.25) (layer "B.Cu") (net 29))
 (segment (start 123.21 101.79) (end 123.21 96.845718) (width 0.25) (layer "B.Cu") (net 29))
 (segment (start 111.5 85.135718) (end 111.5 57.407682) (width 0.25) (layer "B.Cu") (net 29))
 (segment (start 157.5 92.5) (end 146.02 92.5) (width 0.25) (layer "B.Cu") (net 29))
 (segment (start 161.31 96.31) (end 157.5 92.5) (width 0.25) (layer "B.Cu") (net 29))
 (segment (start 118.857202 50.05048) (end 134.95952 50.05048) (width 0.25) (layer "B.Cu") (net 29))
 (segment (start 132.5 92.5) (end 123.21 101.79) (width 0.25) (layer "B.Cu") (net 29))
 (segment (start 146.02 92.5) (end 142.26 96.26) (width 0.25) (layer "B.Cu") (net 29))
 (segment (start 142.26 104.1) (end 142.26 96.26) (width 0.25) (layer "B.Cu") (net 29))
 (segment (start 138.5 92.5) (end 132.5 92.5) (width 0.25) (layer "B.Cu") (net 29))
 (segment (start 153.69 48) (end 144.63 48) (width 0.25) (layer "B.Cu") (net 28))
 (segment (start 144.63 48) (end 144.51 48.12) (width 0.25) (layer "B.Cu") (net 28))
 (segment (start 122.03125 73.02243) (end 122.03125 92.07243) (width 0.25) (layer "F.Cu") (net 6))
 (segment (start 144.5 51) (end 146.55048 48.94952) (width 0.25) (layer "F.Cu") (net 6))
 (segment (start 146.55048 46.686198) (end 139.43 39.565717) (width 0.25) (layer "F.Cu") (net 6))
 (segment (start 122.03125 53.97243) (end 125.00368 51) (width 0.25) (layer "F.Cu") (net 6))
 (segment (start 122.03125 53.97243) (end 122.03125 73.02243) (width 0.25) (layer "F.Cu") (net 6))
 (segment (start 125.00368 51) (end 144.5 51) (width 0.25) (layer "F.Cu") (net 6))
 (segment (start 139.43 39.565717) (end 139.43 32.88) (width 0.25) (layer "F.Cu") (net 6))
 (segment (start 146.55048 48.94952) (end 146.55048 46.686198) (width 0.25) (layer "F.Cu") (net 6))
 (segment (start 141.08125 53.97243) (end 143.52757 53.97243) (width 0.25) (layer "F.Cu") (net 9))
 (segment (start 141.08125 73.02243) (end 141.08125 92.07243) (width 0.25) (layer "F.Cu") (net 9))
 (segment (start 141.08125 73.02243) (end 141.08125 53.97243) (width 0.25) (layer "F.Cu") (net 9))
 (segment (start 141.97 41.47) (end 141.97 32.88) (width 0.25) (layer "F.Cu") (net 9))
 (segment (start 147 46.5) (end 141.97 41.47) (width 0.25) (layer "F.Cu") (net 9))
 (segment (start 147 50.5) (end 147 46.5) (width 0.25) (layer "F.Cu") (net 9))
 (segment (start 143.52757 53.97243) (end 147 50.5) (width 0.25) (layer "F.Cu") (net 9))
 (segment (start 163.5 43.62868) (end 164.75 42.37868) (width 0.25) (layer "F.Cu") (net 4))
 (segment (start 151.635718 50.5) (end 144.51 43.374282) (width 0.25) (layer "F.Cu") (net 4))
 (segment (start 160.13125 73.02243) (end 160.13125 53.97243) (width 0.25) (layer "F.Cu") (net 4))
 (segment (start 163.5 50.5) (end 151.635718 50.5) (width 0.25) (layer "F.Cu") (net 4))
 (segment (start 160.13125 73.02243) (end 160.13125 92.07243) (width 0.25) (layer "F.Cu") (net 4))
 (segment (start 163.5 50.60368) (end 163.5 50.5) (width 0.25) (layer "F.Cu") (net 4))
 (segment (start 163.5 50.5) (end 163.5 43.62868) (width 0.25) (layer "F.Cu") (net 4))
 (segment (start 160.13125 53.97243) (end 163.5 50.60368) (width 0.25) (layer "F.Cu") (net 4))
 (segment (start 144.51 43.374282) (end 144.51 32.88) (width 0.25) (layer "F.Cu") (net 4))
 (segment (start 126 28.53) (end 126 28.5) (width 0.25) (layer "F.Cu") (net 3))
 (segment (start 126 28.5) (end 127.92 26.58) (width 0.25) (layer "F.Cu") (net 3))
 (segment (start 121.65 32.88) (end 126 28.53) (width 0.25) (layer "F.Cu") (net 3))
 (segment (start 127.92 26.58) (end 127.92 23.4) (width 0.25) (layer "F.Cu") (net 3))
 (segment (start 141.00102 39.87868) (end 133.225489 47.654211) (width 0.25) (layer "B.Cu") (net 3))
 (segment (start 120.59096 49.60096) (end 119.11 48.12) (width 0.25) (layer "B.Cu") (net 3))
 (segment (start 133.225489 47.654211) (end 133.225489 48.294811) (width 0.25) (layer "B.Cu") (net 3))
 (segment (start 150.25 39.87868) (end 141.00102 39.87868) (width 0.25) (layer "B.Cu") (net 3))
 (segment (start 133.225489 48.294811) (end 131.91934 49.60096) (width 0.25) (layer "B.Cu") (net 3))
 (segment (start 131.91934 49.60096) (end 120.59096 49.60096) (width 0.25) (layer "B.Cu") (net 3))
 (segment (start 124.19 48.12) (end 125.38 46.93) (width 0.25) (layer "B.Cu") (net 14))
 (segment (start 125.38 46.93) (end 125.38 23.4) (width 0.25) (layer "B.Cu") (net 14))
 (segment (start 140.09132 42.37868) (end 134.35 48.12) (width 0.25) (layer "B.Cu") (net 2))
 (segment (start 150.25 42.37868) (end 140.09132 42.37868) (width 0.25) (layer "B.Cu") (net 2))
 (segment (start 150.25 37.37868) (end 142.55132 37.37868) (width 0.25) (layer "B.Cu") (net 1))
 (segment (start 142.55132 37.37868) (end 131.81 48.12) (width 0.25) (layer "B.Cu") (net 1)))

